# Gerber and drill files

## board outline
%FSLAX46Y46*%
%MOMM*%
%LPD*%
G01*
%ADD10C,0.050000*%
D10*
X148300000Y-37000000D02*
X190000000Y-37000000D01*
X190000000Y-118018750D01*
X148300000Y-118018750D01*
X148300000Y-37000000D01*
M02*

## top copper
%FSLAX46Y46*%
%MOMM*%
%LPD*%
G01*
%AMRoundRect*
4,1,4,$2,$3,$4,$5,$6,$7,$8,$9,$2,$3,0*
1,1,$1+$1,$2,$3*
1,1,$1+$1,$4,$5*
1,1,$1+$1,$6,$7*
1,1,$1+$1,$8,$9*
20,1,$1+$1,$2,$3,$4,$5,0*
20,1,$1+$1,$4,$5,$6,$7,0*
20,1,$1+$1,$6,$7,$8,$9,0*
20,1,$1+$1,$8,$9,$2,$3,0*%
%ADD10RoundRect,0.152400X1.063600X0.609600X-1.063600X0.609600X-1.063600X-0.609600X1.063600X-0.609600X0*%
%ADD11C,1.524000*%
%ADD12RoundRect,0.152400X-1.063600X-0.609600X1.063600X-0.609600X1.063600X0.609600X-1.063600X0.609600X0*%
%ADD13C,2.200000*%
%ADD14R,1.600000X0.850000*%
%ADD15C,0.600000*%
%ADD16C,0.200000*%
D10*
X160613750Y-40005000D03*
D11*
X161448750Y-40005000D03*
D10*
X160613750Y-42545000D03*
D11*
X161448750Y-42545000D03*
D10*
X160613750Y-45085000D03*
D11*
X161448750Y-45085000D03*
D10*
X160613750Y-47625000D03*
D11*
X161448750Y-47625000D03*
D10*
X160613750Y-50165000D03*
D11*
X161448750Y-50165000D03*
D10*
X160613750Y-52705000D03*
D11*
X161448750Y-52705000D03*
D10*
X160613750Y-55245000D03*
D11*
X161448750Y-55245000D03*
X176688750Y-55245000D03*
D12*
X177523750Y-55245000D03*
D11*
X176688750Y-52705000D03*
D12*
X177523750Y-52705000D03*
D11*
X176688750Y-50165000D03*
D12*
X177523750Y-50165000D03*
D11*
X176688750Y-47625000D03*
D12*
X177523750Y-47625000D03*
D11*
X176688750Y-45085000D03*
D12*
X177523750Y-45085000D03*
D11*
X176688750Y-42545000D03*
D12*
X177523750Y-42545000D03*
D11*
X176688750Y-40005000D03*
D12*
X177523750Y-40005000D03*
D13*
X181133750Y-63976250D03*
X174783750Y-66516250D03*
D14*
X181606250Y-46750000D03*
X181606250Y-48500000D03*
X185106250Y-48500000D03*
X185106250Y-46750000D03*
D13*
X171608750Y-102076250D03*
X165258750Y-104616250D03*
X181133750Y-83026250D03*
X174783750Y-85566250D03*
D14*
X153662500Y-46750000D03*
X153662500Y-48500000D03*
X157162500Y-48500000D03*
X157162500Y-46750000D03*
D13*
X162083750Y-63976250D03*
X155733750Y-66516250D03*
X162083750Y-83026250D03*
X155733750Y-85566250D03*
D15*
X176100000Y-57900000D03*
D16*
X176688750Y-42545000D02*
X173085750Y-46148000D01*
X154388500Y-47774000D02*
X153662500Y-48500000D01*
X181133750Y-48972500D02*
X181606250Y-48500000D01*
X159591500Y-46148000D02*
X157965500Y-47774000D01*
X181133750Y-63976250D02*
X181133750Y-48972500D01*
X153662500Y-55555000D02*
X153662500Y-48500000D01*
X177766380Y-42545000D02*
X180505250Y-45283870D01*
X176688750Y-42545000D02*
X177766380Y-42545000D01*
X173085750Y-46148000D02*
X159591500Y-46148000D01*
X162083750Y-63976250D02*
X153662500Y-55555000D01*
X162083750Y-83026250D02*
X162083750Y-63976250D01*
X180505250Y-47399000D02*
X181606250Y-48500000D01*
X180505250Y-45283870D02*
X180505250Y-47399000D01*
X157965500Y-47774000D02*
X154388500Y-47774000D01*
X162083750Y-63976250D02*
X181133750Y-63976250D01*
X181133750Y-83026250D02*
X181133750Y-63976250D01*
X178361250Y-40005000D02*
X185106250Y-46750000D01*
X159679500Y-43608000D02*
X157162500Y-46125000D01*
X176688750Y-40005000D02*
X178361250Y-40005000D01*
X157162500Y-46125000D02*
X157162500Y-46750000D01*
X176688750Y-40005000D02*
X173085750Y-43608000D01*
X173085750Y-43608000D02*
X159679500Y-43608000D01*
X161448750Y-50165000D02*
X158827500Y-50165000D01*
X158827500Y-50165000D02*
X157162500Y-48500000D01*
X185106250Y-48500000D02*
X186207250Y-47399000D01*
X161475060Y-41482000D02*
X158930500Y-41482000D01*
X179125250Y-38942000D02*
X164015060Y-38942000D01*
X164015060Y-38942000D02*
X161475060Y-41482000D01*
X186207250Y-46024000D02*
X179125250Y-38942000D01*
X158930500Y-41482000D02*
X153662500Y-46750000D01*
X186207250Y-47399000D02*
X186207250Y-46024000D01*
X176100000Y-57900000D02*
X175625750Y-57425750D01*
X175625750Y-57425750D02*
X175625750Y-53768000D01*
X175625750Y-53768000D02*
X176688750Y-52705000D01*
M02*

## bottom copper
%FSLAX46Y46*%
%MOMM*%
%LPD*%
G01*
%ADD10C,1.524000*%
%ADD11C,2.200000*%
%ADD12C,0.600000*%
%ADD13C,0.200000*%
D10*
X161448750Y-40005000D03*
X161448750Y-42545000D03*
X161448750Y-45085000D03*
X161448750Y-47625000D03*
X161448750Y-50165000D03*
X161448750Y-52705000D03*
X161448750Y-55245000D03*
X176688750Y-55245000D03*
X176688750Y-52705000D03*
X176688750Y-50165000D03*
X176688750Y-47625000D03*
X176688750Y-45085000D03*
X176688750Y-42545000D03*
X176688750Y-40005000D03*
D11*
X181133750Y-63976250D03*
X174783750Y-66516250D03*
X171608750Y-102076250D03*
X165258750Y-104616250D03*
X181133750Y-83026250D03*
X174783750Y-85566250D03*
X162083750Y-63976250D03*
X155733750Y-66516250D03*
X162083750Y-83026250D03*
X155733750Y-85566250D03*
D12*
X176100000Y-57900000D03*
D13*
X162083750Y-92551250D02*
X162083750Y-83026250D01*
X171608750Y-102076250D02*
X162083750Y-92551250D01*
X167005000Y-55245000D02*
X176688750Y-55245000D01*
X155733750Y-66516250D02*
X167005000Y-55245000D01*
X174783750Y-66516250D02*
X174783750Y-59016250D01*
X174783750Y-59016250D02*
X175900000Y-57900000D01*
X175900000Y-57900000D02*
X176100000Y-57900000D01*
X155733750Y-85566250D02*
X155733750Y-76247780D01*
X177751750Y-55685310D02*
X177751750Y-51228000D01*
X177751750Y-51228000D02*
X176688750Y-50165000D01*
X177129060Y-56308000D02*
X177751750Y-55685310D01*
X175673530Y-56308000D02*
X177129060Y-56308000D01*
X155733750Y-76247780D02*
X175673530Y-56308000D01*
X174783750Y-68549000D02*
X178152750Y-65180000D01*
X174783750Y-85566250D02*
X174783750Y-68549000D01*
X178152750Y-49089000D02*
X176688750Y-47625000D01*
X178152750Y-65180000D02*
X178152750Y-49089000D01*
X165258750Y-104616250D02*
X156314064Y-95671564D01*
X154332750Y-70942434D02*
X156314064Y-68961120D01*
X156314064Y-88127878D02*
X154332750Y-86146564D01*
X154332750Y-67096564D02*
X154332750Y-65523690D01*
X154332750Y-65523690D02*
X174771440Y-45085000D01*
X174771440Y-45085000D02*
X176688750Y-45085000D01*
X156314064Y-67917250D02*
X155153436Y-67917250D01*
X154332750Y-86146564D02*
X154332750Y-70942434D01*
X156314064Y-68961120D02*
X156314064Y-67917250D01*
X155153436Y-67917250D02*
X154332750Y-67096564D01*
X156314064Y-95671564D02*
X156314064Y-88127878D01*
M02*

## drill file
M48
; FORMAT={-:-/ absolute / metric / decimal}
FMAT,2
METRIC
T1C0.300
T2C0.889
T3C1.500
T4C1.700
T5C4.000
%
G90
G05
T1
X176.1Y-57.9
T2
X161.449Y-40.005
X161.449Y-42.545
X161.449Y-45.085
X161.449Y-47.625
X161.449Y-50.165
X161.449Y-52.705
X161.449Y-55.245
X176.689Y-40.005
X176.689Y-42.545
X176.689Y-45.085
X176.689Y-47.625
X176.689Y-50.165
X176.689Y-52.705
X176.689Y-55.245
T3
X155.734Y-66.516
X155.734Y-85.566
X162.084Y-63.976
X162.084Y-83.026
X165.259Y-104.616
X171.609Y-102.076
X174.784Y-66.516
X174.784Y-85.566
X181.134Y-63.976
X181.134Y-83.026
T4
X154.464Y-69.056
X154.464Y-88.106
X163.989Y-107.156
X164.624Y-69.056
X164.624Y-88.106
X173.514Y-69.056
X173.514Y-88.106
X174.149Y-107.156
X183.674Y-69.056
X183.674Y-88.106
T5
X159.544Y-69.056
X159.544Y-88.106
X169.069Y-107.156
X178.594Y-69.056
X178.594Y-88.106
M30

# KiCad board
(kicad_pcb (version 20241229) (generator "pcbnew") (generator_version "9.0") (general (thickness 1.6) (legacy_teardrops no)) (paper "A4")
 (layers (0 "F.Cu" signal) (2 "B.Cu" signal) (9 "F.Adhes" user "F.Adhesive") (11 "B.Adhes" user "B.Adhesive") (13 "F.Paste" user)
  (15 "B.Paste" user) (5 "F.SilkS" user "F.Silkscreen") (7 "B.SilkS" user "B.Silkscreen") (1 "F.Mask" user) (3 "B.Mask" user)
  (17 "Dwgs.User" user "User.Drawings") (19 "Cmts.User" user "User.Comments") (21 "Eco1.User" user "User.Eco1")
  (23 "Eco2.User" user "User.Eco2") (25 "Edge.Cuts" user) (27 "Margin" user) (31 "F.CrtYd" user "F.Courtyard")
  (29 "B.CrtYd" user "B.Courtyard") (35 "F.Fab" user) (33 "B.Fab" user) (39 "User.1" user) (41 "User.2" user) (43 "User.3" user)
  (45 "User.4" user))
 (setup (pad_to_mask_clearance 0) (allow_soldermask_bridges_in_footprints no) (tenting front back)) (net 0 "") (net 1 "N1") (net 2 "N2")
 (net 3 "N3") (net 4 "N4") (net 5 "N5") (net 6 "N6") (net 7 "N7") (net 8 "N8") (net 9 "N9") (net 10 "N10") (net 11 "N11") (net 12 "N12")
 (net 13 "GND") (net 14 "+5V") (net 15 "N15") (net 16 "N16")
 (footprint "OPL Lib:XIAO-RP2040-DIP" (layer "F.Cu") (at 169.06875 47.625)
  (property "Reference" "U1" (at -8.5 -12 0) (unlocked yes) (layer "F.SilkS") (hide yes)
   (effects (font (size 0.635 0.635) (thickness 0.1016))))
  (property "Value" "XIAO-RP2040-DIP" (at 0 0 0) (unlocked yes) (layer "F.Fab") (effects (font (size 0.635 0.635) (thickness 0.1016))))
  (pad "1" smd roundrect (at -8.455 -7.62 180) (size 2.432 1.524) (layers "F.Cu" "F.Mask") (roundrect_rratio 0.1) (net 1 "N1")
   (thermal_bridge_angle 45))
  (pad "1" thru_hole circle (at -7.62 -7.62 180) (size 1.524 1.524) (drill 0.889) (layers "*.Cu" "*.Mask") (remove_unused_layers no)
   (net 1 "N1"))
  (pad "2" smd roundrect (at -8.455 -5.08 180) (size 2.432 1.524) (layers "F.Cu" "F.Mask") (roundrect_rratio 0.1) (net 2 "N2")
   (thermal_bridge_angle 45))
  (pad "2" thru_hole circle (at -7.62 -5.08 180) (size 1.524 1.524) (drill 0.889) (layers "*.Cu" "*.Mask") (remove_unused_layers no)
   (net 2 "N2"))
  (pad "3" smd roundrect (at -8.455 -2.54 180) (size 2.432 1.524) (layers "F.Cu" "F.Mask") (roundrect_rratio 0.1) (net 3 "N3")
   (thermal_bridge_angle 45))
  (pad "3" thru_hole circle (at -7.62 -2.54 180) (size 1.524 1.524) (drill 0.889) (layers "*.Cu" "*.Mask") (remove_unused_layers no)
   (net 3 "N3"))
  (pad "4" smd roundrect (at -8.455 0 180) (size 2.432 1.524) (layers "F.Cu" "F.Mask") (roundrect_rratio 0.1) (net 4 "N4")
   (thermal_bridge_angle 45))
  (pad "4" thru_hole circle (at -7.62 0 180) (size 1.524 1.524) (drill 0.889) (layers "*.Cu" "*.Mask") (remove_unused_layers no)
   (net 4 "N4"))
  (pad "5" smd roundrect (at -8.455 2.54 180) (size 2.432 1.524) (layers "F.Cu" "F.Mask") (roundrect_rratio 0.1) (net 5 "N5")
   (thermal_bridge_angle 45))
  (pad "5" thru_hole circle (at -7.62 2.54 180) (size 1.524 1.524) (drill 0.889) (layers "*.Cu" "*.Mask") (remove_unused_layers no)
   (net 5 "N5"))
  (pad "6" smd roundrect (at -8.455 5.08 180) (size 2.432 1.524) (layers "F.Cu" "F.Mask") (roundrect_rratio 0.1) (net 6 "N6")
   (thermal_bridge_angle 45))
  (pad "6" thru_hole circle (at -7.62 5.08 180) (size 1.524 1.524) (drill 0.889) (layers "*.Cu" "*.Mask") (remove_unused_layers no)
   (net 6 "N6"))
  (pad "7" smd roundrect (at -8.455 7.62 180) (size 2.432 1.524) (layers "F.Cu" "F.Mask") (roundrect_rratio 0.1) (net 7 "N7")
   (thermal_bridge_angle 45))
  (pad "7" thru_hole circle (at -7.62 7.62 180) (size 1.524 1.524) (drill 0.889) (layers "*.Cu" "*.Mask") (remove_unused_layers no)
   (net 7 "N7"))
  (pad "8" thru_hole circle (at 7.62 7.62) (size 1.524 1.524) (drill 0.889) (layers "*.Cu" "*.Mask") (remove_unused_layers no) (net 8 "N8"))
  (pad "8" smd roundrect (at 8.455 7.62) (size 2.432 1.524) (layers "F.Cu" "F.Mask") (roundrect_rratio 0.1) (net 8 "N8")
   (thermal_bridge_angle 45))
  (pad "9" thru_hole circle (at 7.62 5.08) (size 1.524 1.524) (drill 0.889) (layers "*.Cu" "*.Mask") (remove_unused_layers no) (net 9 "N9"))
  (pad "9" smd roundrect (at 8.455 5.08) (size 2.432 1.524) (layers "F.Cu" "F.Mask") (roundrect_rratio 0.1) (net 9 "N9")
   (thermal_bridge_angle 45))
  (pad "10" thru_hole circle (at 7.62 2.54) (size 1.524 1.524) (drill 0.889) (layers "*.Cu" "*.Mask") (remove_unused_layers no)
   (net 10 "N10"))
  (pad "10" smd roundrect (at 8.455 2.54) (size 2.432 1.524) (layers "F.Cu" "F.Mask") (roundrect_rratio 0.1) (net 10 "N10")
   (thermal_bridge_angle 45))
  (pad "11" thru_hole circle (at 7.62 0) (size 1.524 1.524) (drill 0.889) (layers "*.Cu" "*.Mask") (remove_unused_layers no) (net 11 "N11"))
  (pad "11" smd roundrect (at 8.455 0) (size 2.432 1.524) (layers "F.Cu" "F.Mask") (roundrect_rratio 0.1) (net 11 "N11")
   (thermal_bridge_angle 45))
  (pad "12" thru_hole circle (at 7.62 -2.54) (size 1.524 1.524) (drill 0.889) (layers "*.Cu" "*.Mask") (remove_unused_layers no)
   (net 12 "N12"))
  (pad "12" smd roundrect (at 8.455 -2.54) (size 2.432 1.524) (layers "F.Cu" "F.Mask") (roundrect_rratio 0.1) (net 12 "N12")
   (thermal_bridge_angle 45))
  (pad "13" thru_hole circle (at 7.62 -5.08) (size 1.524 1.524) (drill 0.889) (layers "*.Cu" "*.Mask") (remove_unused_layers no)
   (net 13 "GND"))
  (pad "13" smd roundrect (at 8.455 -5.08) (size 2.432 1.524) (layers "F.Cu" "F.Mask") (roundrect_rratio 0.1) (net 13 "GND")
   (thermal_bridge_angle 45))
  (pad "14" thru_hole circle (at 7.62 -7.62) (size 1.524 1.524) (drill 0.889) (layers "*.Cu" "*.Mask") (remove_unused_layers no)
   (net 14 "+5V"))
  (pad "14" smd roundrect (at 8.455 -7.62) (size 2.432 1.524) (layers "F.Cu" "F.Mask") (roundrect_rratio 0.1) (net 14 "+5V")
   (thermal_bridge_angle 45)))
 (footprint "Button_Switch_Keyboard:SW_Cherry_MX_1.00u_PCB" (layer "F.Cu") (at 181.13375 63.97625)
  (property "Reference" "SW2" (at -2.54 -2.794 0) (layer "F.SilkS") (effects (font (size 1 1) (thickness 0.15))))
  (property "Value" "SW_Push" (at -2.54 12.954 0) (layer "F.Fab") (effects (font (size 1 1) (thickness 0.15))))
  (pad "" np_thru_hole circle (at -7.62 5.08) (size 1.7 1.7) (drill 1.7) (layers "*.Cu" "*.Mask"))
  (pad "" np_thru_hole circle (at -2.54 5.08) (size 4 4) (drill 4) (layers "*.Cu" "*.Mask"))
  (pad "" np_thru_hole circle (at 2.54 5.08) (size 1.7 1.7) (drill 1.7) (layers "*.Cu" "*.Mask"))
  (pad "1" thru_hole circle (at 0 0) (size 2.2 2.2) (drill 1.5) (layers "*.Cu" "*.Mask") (remove_unused_layers no) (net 13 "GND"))
  (pad "2" thru_hole circle (at -6.35 2.54) (size 2.2 2.2) (drill 1.5) (layers "*.Cu" "*.Mask") (remove_unused_layers no) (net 9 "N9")))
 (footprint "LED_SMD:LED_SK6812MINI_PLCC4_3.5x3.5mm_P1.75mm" (layer "F.Cu") (at 183.35625 47.625)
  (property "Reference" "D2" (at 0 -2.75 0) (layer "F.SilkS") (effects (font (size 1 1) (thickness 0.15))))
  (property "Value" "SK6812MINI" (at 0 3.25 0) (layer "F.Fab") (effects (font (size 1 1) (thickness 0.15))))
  (pad "1" smd rect (at -1.75 -0.875) (size 1.6 0.85) (layers "F.Cu" "F.Mask" "F.Paste") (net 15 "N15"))
  (pad "2" smd rect (at -1.75 0.875) (size 1.6 0.85) (layers "F.Cu" "F.Mask" "F.Paste") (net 13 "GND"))
  (pad "3" smd rect (at 1.75 0.875) (size 1.6 0.85) (layers "F.Cu" "F.Mask" "F.Paste") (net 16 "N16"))
  (pad "4" smd rect (at 1.75 -0.875) (size 1.6 0.85) (layers "F.Cu" "F.Mask" "F.Paste") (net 14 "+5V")))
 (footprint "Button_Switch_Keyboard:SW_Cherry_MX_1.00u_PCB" (layer "F.Cu") (at 171.60875 102.07625)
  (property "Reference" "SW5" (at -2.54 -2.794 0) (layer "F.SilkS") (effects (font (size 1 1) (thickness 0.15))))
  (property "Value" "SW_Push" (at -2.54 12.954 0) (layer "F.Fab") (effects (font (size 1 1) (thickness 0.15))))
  (pad "" np_thru_hole circle (at -7.62 5.08) (size 1.7 1.7) (drill 1.7) (layers "*.Cu" "*.Mask"))
  (pad "" np_thru_hole circle (at -2.54 5.08) (size 4 4) (drill 4) (layers "*.Cu" "*.Mask"))
  (pad "" np_thru_hole circle (at 2.54 5.08) (size 1.7 1.7) (drill 1.7) (layers "*.Cu" "*.Mask"))
  (pad "1" thru_hole circle (at 0 0) (size 2.2 2.2) (drill 1.5) (layers "*.Cu" "*.Mask") (remove_unused_layers no) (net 13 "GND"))
  (pad "2" thru_hole circle (at -6.35 2.54) (size 2.2 2.2) (drill 1.5) (layers "*.Cu" "*.Mask") (remove_unused_layers no) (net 12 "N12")))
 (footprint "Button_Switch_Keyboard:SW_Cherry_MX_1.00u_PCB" (layer "F.Cu") (at 181.13375 83.02625)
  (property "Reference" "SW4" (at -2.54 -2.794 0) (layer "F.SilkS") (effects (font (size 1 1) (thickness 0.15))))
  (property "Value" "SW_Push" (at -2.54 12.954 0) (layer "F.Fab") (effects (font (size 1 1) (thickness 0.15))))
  (pad "" np_thru_hole circle (at -7.62 5.08) (size 1.7 1.7) (drill 1.7) (layers "*.Cu" "*.Mask"))
  (pad "" np_thru_hole circle (at -2.54 5.08) (size 4 4) (drill 4) (layers "*.Cu" "*.Mask"))
  (pad "" np_thru_hole circle (at 2.54 5.08) (size 1.7 1.7) (drill 1.7) (layers "*.Cu" "*.Mask"))
  (pad "1" thru_hole circle (at 0 0) (size 2.2 2.2) (drill 1.5) (layers "*.Cu" "*.Mask") (remove_unused_layers no) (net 13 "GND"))
  (pad "2" thru_hole circle (at -6.35 2.54) (size 2.2 2.2) (drill 1.5) (layers "*.Cu" "*.Mask") (remove_unused_layers no) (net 11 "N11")))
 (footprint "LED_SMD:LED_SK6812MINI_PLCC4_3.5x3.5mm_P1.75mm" (layer "F.Cu") (at 155.4125 47.625)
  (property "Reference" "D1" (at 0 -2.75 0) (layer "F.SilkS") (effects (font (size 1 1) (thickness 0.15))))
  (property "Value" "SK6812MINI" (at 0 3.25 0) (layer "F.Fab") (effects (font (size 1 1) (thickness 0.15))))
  (pad "1" smd rect (at -1.75 -0.875) (size 1.6 0.85) (layers "F.Cu" "F.Mask" "F.Paste") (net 16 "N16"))
  (pad "2" smd rect (at -1.75 0.875) (size 1.6 0.85) (layers "F.Cu" "F.Mask" "F.Paste") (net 13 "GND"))
  (pad "3" smd rect (at 1.75 0.875) (size 1.6 0.85) (layers "F.Cu" "F.Mask" "F.Paste") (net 5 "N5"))
  (pad "4" smd rect (at 1.75 -0.875) (size 1.6 0.85) (layers "F.Cu" "F.Mask" "F.Paste") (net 14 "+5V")))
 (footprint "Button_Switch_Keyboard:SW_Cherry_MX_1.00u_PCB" (layer "F.Cu") (at 162.08375 63.97625)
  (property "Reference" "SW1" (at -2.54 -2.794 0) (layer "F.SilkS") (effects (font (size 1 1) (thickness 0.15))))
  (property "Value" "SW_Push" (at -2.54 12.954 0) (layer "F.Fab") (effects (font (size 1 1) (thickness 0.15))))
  (pad "" np_thru_hole circle (at -7.62 5.08) (size 1.7 1.7) (drill 1.7) (layers "*.Cu" "*.Mask"))
  (pad "" np_thru_hole circle (at -2.54 5.08) (size 4 4) (drill 4) (layers "*.Cu" "*.Mask"))
  (pad "" np_thru_hole circle (at 2.54 5.08) (size 1.7 1.7) (drill 1.7) (layers "*.Cu" "*.Mask"))
  (pad "1" thru_hole circle (at 0 0) (size 2.2 2.2) (drill 1.5) (layers "*.Cu" "*.Mask") (remove_unused_layers no) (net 13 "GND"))
  (pad "2" thru_hole circle (at -6.35 2.54) (size 2.2 2.2) (drill 1.5) (layers "*.Cu" "*.Mask") (remove_unused_layers no) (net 8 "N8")))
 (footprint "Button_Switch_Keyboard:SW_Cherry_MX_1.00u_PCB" (layer "F.Cu") (at 162.08375 83.02625)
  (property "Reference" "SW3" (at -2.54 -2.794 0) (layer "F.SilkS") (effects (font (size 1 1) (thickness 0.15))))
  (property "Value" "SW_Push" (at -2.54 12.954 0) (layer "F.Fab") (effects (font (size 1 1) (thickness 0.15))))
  (pad "" np_thru_hole circle (at -7.62 5.08) (size 1.7 1.7) (drill 1.7) (layers "*.Cu" "*.Mask"))
  (pad "" np_thru_hole circle (at -2.54 5.08) (size 4 4) (drill 4) (layers "*.Cu" "*.Mask"))
  (pad "" np_thru_hole circle (at 2.54 5.08) (size 1.7 1.7) (drill 1.7) (layers "*.Cu" "*.Mask"))
  (pad "1" thru_hole circle (at 0 0) (size 2.2 2.2) (drill 1.5) (layers "*.Cu" "*.Mask") (remove_unused_layers no) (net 13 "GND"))
  (pad "2" thru_hole circle (at -6.35 2.54) (size 2.2 2.2) (drill 1.5) (layers "*.Cu" "*.Mask") (remove_unused_layers no) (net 10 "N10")))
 (gr_rect (start 148.3 37) (end 190 118.01875) (stroke (width 0.05) (type default)) (fill no) (layer "Edge.Cuts"))
 (segment (start 176.68875 42.545) (end 173.08575 46.148) (width 0.2) (layer "F.Cu") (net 13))
 (segment (start 154.3885 47.774) (end 153.6625 48.5) (width 0.2) (layer "F.Cu") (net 13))
 (segment (start 181.13375 48.9725) (end 181.60625 48.5) (width 0.2) (layer "F.Cu") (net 13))
 (segment (start 159.5915 46.148) (end 157.9655 47.774) (width 0.2) (layer "F.Cu") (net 13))
 (segment (start 181.13375 63.97625) (end 181.13375 48.9725) (width 0.2) (layer "F.Cu") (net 13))
 (segment (start 153.6625 55.555) (end 153.6625 48.5) (width 0.2) (layer "F.Cu") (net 13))
 (segment (start 177.76638 42.545) (end 180.50525 45.28387) (width 0.2) (layer "F.Cu") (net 13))
 (segment (start 176.68875 42.545) (end 177.76638 42.545) (width 0.2) (layer "F.Cu") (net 13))
 (segment (start 173.08575 46.148) (end 159.5915 46.148) (width 0.2) (layer "F.Cu") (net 13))
 (segment (start 162.08375 63.97625) (end 153.6625 55.555) (width 0.2) (layer "F.Cu") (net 13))
 (segment (start 162.08375 83.02625) (end 162.08375 63.97625) (width 0.2) (layer "F.Cu") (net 13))
 (segment (start 180.50525 47.399) (end 181.60625 48.5) (width 0.2) (layer "F.Cu") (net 13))
 (segment (start 180.50525 45.28387) (end 180.50525 47.399) (width 0.2) (layer "F.Cu") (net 13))
 (segment (start 157.9655 47.774) (end 154.3885 47.774) (width 0.2) (layer "F.Cu") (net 13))
 (segment (start 162.08375 63.97625) (end 181.13375 63.97625) (width 0.2) (layer "F.Cu") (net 13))
 (segment (start 181.13375 83.02625) (end 181.13375 63.97625) (width 0.2) (layer "F.Cu") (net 13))
 (segment (start 162.08375 92.55125) (end 162.08375 83.02625) (width 0.2) (layer "B.Cu") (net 13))
 (segment (start 171.60875 102.07625) (end 162.08375 92.55125) (width 0.2) (layer "B.Cu") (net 13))
 (segment (start 178.36125 40.005) (end 185.10625 46.75) (width 0.2) (layer "F.Cu") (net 14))
 (segment (start 159.6795 43.608) (end 157.1625 46.125) (width 0.2) (layer "F.Cu") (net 14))
 (segment (start 176.68875 40.005) (end 178.36125 40.005) (width 0.2) (layer "F.Cu") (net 14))
 (segment (start 157.1625 46.125) (end 157.1625 46.75) (width 0.2) (layer "F.Cu") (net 14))
 (segment (start 176.68875 40.005) (end 173.08575 43.608) (width 0.2) (layer "F.Cu") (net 14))
 (segment (start 173.08575 43.608) (end 159.6795 43.608) (width 0.2) (layer "F.Cu") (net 14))
 (segment (start 161.44875 50.165) (end 158.8275 50.165) (width 0.2) (layer "F.Cu") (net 5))
 (segment (start 158.8275 50.165) (end 157.1625 48.5) (width 0.2) (layer "F.Cu") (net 5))
 (segment (start 185.10625 48.5) (end 186.20725 47.399) (width 0.2) (layer "F.Cu") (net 16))
 (segment (start 161.47506 41.482) (end 158.9305 41.482) (width 0.2) (layer "F.Cu") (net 16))
 (segment (start 179.12525 38.942) (end 164.01506 38.942) (width 0.2) (layer "F.Cu") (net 16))
 (segment (start 164.01506 38.942) (end 161.47506 41.482) (width 0.2) (layer "F.Cu") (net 16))
 (segment (start 186.20725 46.024) (end 179.12525 38.942) (width 0.2) (layer "F.Cu") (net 16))
 (segment (start 158.9305 41.482) (end 153.6625 46.75) (width 0.2) (layer "F.Cu") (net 16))
 (segment (start 186.20725 47.399) (end 186.20725 46.024) (width 0.2) (layer "F.Cu") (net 16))
 (segment (start 167.005 55.245) (end 176.68875 55.245) (width 0.2) (layer "B.Cu") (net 8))
 (segment (start 155.73375 66.51625) (end 167.005 55.245) (width 0.2) (layer "B.Cu") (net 8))
 (segment (start 176.1 57.9) (end 175.62575 57.42575) (width 0.2) (layer "F.Cu") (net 9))
 (segment (start 175.62575 57.42575) (end 175.62575 53.768) (width 0.2) (layer "F.Cu") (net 9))
 (segment (start 175.62575 53.768) (end 176.68875 52.705) (width 0.2) (layer "F.Cu") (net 9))
 (via (at 176.1 57.9) (size 0.6) (drill 0.3) (layers "F.Cu" "B.Cu") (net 9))
 (segment (start 174.78375 66.51625) (end 174.78375 59.01625) (width 0.2) (layer "B.Cu") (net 9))
 (segment (start 174.78375 59.01625) (end 175.9 57.9) (width 0.2) (layer "B.Cu") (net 9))
 (segment (start 175.9 57.9) (end 176.1 57.9) (width 0.2) (layer "B.Cu") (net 9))
 (segment (start 155.73375 85.56625) (end 155.73375 76.24778) (width 0.2) (layer "B.Cu") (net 10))
 (segment (start 177.75175 55.68531) (end 177.75175 51.228) (width 0.2) (layer "B.Cu") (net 10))
 (segment (start 177.75175 51.228) (end 176.68875 50.165) (width 0.2) (layer "B.Cu") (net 10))
 (segment (start 177.12906 56.308) (end 177.75175 55.68531) (width 0.2) (layer "B.Cu") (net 10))
 (segment (start 175.67353 56.308) (end 177.12906 56.308) (width 0.2) (layer "B.Cu") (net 10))
 (segment (start 155.73375 76.24778) (end 175.67353 56.308) (width 0.2) (layer "B.Cu") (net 10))
 (segment (start 174.78375 68.549) (end 178.15275 65.18) (width 0.2) (layer "B.Cu") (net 11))
 (segment (start 174.78375 85.56625) (end 174.78375 68.549) (width 0.2) (layer "B.Cu") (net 11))
 (segment (start 178.15275 49.089) (end 176.68875 47.625) (width 0.2) (layer "B.Cu") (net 11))
 (segment (start 178.15275 65.18) (end 178.15275 49.089) (width 0.2) (layer "B.Cu") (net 11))
 (segment (start 165.25875 104.61625) (end 156.314064 95.671564) (width 0.2) (layer "B.Cu") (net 12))
 (segment (start 154.33275 70.942434) (end 156.314064 68.96112) (width 0.2) (layer "B.Cu") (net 12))
 (segment (start 156.314064 88.127878) (end 154.33275 86.146564) (width 0.2) (layer "B.Cu") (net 12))
 (segment (start 154.33275 67.096564) (end 154.33275 65.52369) (width 0.2) (layer "B.Cu") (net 12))
 (segment (start 154.33275 65.52369) (end 174.77144 45.085) (width 0.2) (layer "B.Cu") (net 12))
 (segment (start 174.77144 45.085) (end 176.68875 45.085) (width 0.2) (layer "B.Cu") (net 12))
 (segment (start 156.314064 67.91725) (end 155.153436 67.91725) (width 0.2) (layer "B.Cu") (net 12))
 (segment (start 154.33275 86.146564) (end 154.33275 70.942434) (width 0.2) (layer "B.Cu") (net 12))
 (segment (start 156.314064 68.96112) (end 156.314064 67.91725) (width 0.2) (layer "B.Cu") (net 12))
 (segment (start 155.153436 67.91725) (end 154.33275 67.096564) (width 0.2) (layer "B.Cu") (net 12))
 (segment (start 156.314064 95.671564) (end 156.314064 88.127878) (width 0.2) (layer "B.Cu") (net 12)))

